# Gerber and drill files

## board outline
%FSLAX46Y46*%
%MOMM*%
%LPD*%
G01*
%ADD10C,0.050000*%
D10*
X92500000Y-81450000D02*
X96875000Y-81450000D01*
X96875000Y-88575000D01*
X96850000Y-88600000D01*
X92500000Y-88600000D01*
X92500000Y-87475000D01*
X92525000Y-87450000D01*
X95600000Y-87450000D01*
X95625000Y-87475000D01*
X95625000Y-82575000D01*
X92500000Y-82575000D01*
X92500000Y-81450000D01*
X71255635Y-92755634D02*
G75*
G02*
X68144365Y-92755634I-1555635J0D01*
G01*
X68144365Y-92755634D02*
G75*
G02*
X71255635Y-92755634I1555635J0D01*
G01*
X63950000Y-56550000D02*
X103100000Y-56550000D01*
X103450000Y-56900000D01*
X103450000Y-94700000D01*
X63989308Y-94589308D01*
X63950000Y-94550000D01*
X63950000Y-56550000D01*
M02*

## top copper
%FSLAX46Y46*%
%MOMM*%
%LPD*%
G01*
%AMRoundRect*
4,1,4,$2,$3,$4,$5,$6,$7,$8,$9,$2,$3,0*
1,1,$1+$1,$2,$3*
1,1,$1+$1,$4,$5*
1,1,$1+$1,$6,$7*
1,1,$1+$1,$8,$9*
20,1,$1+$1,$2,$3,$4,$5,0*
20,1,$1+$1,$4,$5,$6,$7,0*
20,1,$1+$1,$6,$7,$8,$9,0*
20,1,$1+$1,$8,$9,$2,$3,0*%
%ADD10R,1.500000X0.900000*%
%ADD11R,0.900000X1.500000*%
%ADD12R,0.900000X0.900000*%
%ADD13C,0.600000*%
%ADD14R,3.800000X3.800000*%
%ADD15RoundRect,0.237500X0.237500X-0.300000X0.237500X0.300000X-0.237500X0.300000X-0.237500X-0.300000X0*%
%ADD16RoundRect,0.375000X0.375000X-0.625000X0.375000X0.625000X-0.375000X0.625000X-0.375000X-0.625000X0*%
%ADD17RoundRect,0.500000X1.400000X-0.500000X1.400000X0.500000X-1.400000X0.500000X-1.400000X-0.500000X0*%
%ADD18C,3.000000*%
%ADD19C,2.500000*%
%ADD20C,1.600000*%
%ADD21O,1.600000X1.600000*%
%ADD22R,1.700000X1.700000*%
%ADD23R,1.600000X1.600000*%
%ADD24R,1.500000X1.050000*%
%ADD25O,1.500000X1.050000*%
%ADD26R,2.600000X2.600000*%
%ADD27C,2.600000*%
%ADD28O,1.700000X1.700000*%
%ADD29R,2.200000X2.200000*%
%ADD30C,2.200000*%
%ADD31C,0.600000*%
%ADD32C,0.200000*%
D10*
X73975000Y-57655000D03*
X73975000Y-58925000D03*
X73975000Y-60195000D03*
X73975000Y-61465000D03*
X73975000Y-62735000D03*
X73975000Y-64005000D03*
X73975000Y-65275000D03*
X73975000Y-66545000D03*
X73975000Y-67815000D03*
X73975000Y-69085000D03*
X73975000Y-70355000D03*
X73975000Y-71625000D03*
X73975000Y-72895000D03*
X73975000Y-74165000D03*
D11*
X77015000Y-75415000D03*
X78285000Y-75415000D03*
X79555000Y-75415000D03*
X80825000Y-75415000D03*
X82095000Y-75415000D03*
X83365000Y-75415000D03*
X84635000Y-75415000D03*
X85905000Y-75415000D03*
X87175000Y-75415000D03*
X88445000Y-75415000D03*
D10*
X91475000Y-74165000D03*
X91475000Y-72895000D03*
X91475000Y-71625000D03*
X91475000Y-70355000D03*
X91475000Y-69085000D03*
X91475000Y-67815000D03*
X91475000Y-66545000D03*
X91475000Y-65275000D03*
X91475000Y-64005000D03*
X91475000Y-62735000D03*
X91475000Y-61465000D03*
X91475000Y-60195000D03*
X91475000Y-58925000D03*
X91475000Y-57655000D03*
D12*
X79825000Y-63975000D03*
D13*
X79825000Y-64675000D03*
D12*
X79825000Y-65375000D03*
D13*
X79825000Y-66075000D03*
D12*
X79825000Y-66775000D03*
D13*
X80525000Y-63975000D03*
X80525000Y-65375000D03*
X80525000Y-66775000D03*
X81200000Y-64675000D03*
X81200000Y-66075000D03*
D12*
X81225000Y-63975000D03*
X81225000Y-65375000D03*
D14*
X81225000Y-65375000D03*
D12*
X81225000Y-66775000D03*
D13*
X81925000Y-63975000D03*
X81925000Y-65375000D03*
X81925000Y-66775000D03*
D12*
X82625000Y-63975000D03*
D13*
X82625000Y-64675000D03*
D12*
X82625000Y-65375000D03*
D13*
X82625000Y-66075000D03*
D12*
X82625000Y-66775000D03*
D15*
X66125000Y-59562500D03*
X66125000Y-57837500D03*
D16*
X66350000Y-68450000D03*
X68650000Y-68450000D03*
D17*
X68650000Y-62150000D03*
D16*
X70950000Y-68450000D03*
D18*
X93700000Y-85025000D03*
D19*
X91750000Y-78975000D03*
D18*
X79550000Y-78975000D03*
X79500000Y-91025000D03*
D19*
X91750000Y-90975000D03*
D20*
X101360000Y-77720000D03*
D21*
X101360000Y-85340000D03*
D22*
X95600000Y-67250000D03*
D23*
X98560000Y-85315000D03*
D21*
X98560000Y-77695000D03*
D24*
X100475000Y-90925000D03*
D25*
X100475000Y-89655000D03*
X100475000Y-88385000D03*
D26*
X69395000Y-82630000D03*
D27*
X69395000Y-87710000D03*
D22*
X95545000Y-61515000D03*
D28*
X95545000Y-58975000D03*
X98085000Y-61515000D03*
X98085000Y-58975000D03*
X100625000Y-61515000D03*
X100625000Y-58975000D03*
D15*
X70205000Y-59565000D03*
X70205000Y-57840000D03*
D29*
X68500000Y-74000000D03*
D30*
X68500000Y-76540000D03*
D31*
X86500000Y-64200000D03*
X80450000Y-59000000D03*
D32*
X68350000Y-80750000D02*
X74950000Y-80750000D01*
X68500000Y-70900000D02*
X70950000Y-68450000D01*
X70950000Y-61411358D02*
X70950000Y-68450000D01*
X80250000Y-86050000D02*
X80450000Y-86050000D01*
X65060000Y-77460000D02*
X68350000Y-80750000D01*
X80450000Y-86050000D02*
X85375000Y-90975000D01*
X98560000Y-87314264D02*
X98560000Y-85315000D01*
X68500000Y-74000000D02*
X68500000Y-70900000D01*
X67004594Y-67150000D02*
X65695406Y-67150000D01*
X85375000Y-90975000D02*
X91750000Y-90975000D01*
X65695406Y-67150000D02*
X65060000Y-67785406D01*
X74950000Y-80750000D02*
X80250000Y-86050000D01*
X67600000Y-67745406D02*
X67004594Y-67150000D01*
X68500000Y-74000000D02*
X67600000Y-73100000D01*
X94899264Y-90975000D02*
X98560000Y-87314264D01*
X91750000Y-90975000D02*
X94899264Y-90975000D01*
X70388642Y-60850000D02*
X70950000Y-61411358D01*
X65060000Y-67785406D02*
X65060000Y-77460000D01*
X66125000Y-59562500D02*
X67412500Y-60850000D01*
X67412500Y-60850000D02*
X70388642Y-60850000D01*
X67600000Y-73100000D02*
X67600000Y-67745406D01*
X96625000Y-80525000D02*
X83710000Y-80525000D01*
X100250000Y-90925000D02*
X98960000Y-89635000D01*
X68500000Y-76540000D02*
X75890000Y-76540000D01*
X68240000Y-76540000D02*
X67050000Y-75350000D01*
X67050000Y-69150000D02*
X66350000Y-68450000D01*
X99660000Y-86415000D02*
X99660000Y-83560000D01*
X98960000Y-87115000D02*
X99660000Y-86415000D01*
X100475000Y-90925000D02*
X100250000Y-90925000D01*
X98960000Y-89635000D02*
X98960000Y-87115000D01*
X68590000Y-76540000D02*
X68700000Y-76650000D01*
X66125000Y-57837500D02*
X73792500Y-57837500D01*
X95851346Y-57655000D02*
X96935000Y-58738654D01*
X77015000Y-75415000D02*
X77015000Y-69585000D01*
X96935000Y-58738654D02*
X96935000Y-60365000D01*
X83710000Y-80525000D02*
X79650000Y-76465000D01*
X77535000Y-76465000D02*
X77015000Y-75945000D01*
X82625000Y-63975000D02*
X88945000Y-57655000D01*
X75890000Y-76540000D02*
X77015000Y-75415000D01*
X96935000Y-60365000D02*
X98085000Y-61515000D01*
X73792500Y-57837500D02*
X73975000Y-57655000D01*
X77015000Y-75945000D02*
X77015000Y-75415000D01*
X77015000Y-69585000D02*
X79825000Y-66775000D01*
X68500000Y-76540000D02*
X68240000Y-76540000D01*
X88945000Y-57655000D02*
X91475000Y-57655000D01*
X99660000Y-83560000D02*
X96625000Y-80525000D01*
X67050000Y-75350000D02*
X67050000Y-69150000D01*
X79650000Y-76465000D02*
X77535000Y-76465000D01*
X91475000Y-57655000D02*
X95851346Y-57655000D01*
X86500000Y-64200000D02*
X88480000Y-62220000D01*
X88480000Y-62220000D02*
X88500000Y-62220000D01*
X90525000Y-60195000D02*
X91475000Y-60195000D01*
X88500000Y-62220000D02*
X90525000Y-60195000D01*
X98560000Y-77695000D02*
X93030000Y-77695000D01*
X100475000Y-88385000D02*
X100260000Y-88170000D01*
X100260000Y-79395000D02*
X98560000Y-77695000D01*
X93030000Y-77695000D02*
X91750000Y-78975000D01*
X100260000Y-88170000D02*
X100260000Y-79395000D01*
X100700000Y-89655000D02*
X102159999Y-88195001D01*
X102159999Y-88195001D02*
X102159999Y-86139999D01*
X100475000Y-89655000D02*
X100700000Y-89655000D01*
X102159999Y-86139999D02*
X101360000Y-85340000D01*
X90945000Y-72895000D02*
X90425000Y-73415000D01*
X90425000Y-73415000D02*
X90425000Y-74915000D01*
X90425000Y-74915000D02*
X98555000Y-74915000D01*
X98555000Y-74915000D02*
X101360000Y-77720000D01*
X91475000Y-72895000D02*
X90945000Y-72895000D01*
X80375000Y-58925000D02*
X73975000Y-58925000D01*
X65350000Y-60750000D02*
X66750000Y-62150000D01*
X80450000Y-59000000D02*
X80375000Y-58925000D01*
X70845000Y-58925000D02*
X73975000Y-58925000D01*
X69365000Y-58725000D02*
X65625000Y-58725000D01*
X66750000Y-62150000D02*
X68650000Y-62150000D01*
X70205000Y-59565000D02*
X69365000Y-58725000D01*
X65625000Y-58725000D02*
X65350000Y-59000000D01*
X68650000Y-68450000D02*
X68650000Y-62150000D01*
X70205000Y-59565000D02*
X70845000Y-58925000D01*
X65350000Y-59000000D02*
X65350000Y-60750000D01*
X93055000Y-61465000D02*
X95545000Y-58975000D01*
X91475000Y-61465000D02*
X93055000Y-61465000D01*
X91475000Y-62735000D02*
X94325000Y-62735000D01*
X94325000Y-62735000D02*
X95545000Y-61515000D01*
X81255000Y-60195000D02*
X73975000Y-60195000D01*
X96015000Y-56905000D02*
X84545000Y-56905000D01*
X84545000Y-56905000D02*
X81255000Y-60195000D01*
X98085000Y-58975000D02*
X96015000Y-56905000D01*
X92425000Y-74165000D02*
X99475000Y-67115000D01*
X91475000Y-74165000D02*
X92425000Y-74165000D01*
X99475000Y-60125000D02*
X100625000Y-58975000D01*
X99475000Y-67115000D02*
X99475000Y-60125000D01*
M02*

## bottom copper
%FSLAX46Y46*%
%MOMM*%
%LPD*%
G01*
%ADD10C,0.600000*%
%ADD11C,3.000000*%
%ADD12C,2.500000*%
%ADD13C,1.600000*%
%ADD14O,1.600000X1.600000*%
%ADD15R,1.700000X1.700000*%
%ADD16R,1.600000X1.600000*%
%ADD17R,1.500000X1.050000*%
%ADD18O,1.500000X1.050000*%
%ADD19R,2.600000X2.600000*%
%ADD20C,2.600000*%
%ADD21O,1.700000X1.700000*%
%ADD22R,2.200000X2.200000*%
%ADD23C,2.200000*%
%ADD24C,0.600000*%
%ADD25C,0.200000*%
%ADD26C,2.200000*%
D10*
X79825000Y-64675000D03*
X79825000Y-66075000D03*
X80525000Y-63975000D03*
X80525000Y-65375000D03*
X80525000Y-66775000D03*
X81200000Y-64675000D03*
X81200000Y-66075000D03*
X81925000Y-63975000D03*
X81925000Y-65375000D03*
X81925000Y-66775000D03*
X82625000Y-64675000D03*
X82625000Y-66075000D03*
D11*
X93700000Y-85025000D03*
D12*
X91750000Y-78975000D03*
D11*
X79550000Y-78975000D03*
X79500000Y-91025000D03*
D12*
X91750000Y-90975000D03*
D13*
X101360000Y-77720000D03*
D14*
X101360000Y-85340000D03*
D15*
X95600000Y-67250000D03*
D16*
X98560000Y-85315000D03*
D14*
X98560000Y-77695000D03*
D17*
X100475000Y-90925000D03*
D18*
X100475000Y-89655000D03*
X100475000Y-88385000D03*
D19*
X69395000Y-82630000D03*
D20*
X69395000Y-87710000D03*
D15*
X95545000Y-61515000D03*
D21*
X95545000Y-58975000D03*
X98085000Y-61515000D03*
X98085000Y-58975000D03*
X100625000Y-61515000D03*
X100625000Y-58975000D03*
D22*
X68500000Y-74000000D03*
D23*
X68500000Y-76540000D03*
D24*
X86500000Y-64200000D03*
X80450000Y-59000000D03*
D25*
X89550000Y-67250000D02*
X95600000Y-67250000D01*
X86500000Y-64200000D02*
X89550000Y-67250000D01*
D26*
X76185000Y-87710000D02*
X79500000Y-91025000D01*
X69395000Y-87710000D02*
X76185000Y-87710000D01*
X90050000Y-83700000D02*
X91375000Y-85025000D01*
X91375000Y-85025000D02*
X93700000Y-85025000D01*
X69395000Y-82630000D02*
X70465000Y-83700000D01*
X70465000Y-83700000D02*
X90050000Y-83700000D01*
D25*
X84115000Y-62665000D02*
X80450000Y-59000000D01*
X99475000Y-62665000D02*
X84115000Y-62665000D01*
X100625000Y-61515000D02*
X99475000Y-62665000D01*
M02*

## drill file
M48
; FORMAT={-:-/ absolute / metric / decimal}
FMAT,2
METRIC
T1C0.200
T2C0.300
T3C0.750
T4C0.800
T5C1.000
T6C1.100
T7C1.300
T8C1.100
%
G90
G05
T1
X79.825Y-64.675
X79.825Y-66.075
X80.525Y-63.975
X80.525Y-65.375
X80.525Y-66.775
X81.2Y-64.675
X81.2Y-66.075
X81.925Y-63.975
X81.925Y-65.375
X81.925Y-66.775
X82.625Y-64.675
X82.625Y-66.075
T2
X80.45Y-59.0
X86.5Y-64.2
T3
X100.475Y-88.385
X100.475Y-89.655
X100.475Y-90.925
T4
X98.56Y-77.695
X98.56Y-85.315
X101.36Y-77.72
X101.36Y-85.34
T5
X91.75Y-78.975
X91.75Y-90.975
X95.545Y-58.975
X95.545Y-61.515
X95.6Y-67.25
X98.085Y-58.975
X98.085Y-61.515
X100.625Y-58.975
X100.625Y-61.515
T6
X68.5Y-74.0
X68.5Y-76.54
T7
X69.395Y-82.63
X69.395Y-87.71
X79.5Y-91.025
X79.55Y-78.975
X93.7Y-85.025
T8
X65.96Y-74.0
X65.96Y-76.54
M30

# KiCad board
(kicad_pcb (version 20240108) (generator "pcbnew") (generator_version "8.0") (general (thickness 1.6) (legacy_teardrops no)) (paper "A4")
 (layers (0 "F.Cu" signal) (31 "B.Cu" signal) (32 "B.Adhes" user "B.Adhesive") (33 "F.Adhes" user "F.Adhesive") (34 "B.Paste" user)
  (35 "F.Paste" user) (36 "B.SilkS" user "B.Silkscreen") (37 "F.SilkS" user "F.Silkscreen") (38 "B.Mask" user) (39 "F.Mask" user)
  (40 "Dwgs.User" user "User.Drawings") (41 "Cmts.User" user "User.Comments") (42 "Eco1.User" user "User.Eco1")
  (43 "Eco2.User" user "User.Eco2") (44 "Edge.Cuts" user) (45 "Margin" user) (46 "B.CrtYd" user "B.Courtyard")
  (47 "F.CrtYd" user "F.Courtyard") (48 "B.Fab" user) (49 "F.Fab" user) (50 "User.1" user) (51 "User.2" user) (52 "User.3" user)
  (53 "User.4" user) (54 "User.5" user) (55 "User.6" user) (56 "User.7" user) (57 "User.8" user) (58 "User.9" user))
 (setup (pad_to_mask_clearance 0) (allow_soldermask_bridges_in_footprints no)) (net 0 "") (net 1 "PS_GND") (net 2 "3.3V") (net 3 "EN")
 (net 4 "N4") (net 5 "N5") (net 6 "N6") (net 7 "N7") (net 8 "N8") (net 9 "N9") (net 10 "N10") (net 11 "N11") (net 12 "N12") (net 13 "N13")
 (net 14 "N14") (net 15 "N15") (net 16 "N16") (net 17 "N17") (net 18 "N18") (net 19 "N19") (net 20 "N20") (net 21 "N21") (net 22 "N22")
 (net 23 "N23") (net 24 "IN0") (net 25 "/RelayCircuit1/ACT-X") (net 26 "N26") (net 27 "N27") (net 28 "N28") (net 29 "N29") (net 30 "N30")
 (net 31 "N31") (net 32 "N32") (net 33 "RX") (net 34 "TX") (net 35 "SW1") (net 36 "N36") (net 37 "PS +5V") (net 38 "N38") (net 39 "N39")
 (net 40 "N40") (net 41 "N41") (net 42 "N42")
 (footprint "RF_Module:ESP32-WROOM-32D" (layer "F.Cu") (at 82.725 65.905)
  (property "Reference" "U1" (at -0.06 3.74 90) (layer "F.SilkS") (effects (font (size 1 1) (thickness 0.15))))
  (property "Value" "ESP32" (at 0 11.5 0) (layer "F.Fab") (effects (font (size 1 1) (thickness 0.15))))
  (pad "1" smd rect (at -8.75 -8.25) (size 1.5 0.9) (layers "F.Cu" "F.Paste" "F.Mask") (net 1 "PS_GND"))
  (pad "2" smd rect (at -8.75 -6.98) (size 1.5 0.9) (layers "F.Cu" "F.Paste" "F.Mask") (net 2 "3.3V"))
  (pad "3" smd rect (at -8.75 -5.71) (size 1.5 0.9) (layers "F.Cu" "F.Paste" "F.Mask") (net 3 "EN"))
  (pad "4" smd rect (at -8.75 -4.44) (size 1.5 0.9) (layers "F.Cu" "F.Paste" "F.Mask") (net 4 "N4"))
  (pad "5" smd rect (at -8.75 -3.17) (size 1.5 0.9) (layers "F.Cu" "F.Paste" "F.Mask") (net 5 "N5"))
  (pad "6" smd rect (at -8.75 -1.9) (size 1.5 0.9) (layers "F.Cu" "F.Paste" "F.Mask") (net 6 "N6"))
  (pad "7" smd rect (at -8.75 -0.63) (size 1.5 0.9) (layers "F.Cu" "F.Paste" "F.Mask") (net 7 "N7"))
  (pad "8" smd rect (at -8.75 0.64) (size 1.5 0.9) (layers "F.Cu" "F.Paste" "F.Mask") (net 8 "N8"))
  (pad "9" smd rect (at -8.75 1.91) (size 1.5 0.9) (layers "F.Cu" "F.Paste" "F.Mask") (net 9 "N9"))
  (pad "10" smd rect (at -8.75 3.18) (size 1.5 0.9) (layers "F.Cu" "F.Paste" "F.Mask") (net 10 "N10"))
  (pad "11" smd rect (at -8.75 4.45) (size 1.5 0.9) (layers "F.Cu" "F.Paste" "F.Mask") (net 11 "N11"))
  (pad "12" smd rect (at -8.75 5.72) (size 1.5 0.9) (layers "F.Cu" "F.Paste" "F.Mask") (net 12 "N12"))
  (pad "13" smd rect (at -8.75 6.99) (size 1.5 0.9) (layers "F.Cu" "F.Paste" "F.Mask") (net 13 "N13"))
  (pad "14" smd rect (at -8.75 8.26) (size 1.5 0.9) (layers "F.Cu" "F.Paste" "F.Mask") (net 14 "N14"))
  (pad "15" smd rect (at -5.71 9.51 90) (size 1.5 0.9) (layers "F.Cu" "F.Paste" "F.Mask") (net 1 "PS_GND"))
  (pad "16" smd rect (at -4.44 9.51 90) (size 1.5 0.9) (layers "F.Cu" "F.Paste" "F.Mask") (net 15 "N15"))
  (pad "17" smd rect (at -3.17 9.51 90) (size 1.5 0.9) (layers "F.Cu" "F.Paste" "F.Mask") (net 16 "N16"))
  (pad "18" smd rect (at -1.9 9.51 90) (size 1.5 0.9) (layers "F.Cu" "F.Paste" "F.Mask") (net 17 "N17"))
  (pad "19" smd rect (at -0.63 9.51 90) (size 1.5 0.9) (layers "F.Cu" "F.Paste" "F.Mask") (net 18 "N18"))
  (pad "20" smd rect (at 0.64 9.51 90) (size 1.5 0.9) (layers "F.Cu" "F.Paste" "F.Mask") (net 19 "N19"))
  (pad "21" smd rect (at 1.91 9.51 90) (size 1.5 0.9) (layers "F.Cu" "F.Paste" "F.Mask") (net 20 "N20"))
  (pad "22" smd rect (at 3.18 9.51 90) (size 1.5 0.9) (layers "F.Cu" "F.Paste" "F.Mask") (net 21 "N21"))
  (pad "23" smd rect (at 4.45 9.51 90) (size 1.5 0.9) (layers "F.Cu" "F.Paste" "F.Mask") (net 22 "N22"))
  (pad "24" smd rect (at 5.72 9.51 90) (size 1.5 0.9) (layers "F.Cu" "F.Paste" "F.Mask") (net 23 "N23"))
  (pad "25" smd rect (at 8.75 8.26) (size 1.5 0.9) (layers "F.Cu" "F.Paste" "F.Mask") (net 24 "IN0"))
  (pad "26" smd rect (at 8.75 6.99) (size 1.5 0.9) (layers "F.Cu" "F.Paste" "F.Mask") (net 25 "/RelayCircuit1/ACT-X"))
  (pad "27" smd rect (at 8.75 5.72) (size 1.5 0.9) (layers "F.Cu" "F.Paste" "F.Mask") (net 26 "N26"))
  (pad "28" smd rect (at 8.75 4.45) (size 1.5 0.9) (layers "F.Cu" "F.Paste" "F.Mask") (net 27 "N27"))
  (pad "29" smd rect (at 8.75 3.18) (size 1.5 0.9) (layers "F.Cu" "F.Paste" "F.Mask") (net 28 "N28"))
  (pad "30" smd rect (at 8.75 1.91) (size 1.5 0.9) (layers "F.Cu" "F.Paste" "F.Mask") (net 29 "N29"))
  (pad "31" smd rect (at 8.75 0.64) (size 1.5 0.9) (layers "F.Cu" "F.Paste" "F.Mask") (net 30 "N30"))
  (pad "32" smd rect (at 8.75 -0.63) (size 1.5 0.9) (layers "F.Cu" "F.Paste" "F.Mask") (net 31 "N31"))
  (pad "33" smd rect (at 8.75 -1.9) (size 1.5 0.9) (layers "F.Cu" "F.Paste" "F.Mask") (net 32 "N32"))
  (pad "34" smd rect (at 8.75 -3.17) (size 1.5 0.9) (layers "F.Cu" "F.Paste" "F.Mask") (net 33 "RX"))
  (pad "35" smd rect (at 8.75 -4.44) (size 1.5 0.9) (layers "F.Cu" "F.Paste" "F.Mask") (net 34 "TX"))
  (pad "36" smd rect (at 8.75 -5.71) (size 1.5 0.9) (layers "F.Cu" "F.Paste" "F.Mask") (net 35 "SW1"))
  (pad "37" smd rect (at 8.75 -6.98) (size 1.5 0.9) (layers "F.Cu" "F.Paste" "F.Mask") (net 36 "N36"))
  (pad "38" smd rect (at 8.75 -8.25) (size 1.5 0.9) (layers "F.Cu" "F.Paste" "F.Mask") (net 1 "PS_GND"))
  (pad "39" smd rect (at -2.9 -1.93) (size 0.9 0.9) (layers "F.Cu" "F.Paste") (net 1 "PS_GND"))
  (pad "39" thru_hole circle (at -2.9 -1.23) (size 0.6 0.6) (drill 0.2) (layers "*.Cu" "F.Mask") (remove_unused_layers no) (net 1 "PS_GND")
   (zone_connect 2))
  (pad "39" smd rect (at -2.9 -0.53) (size 0.9 0.9) (layers "F.Cu" "F.Paste") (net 1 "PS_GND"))
  (pad "39" thru_hole circle (at -2.9 0.17) (size 0.6 0.6) (drill 0.2) (layers "*.Cu" "F.Mask") (remove_unused_layers no) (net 1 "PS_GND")
   (zone_connect 2))
  (pad "39" smd rect (at -2.9 0.87) (size 0.9 0.9) (layers "F.Cu" "F.Paste") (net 1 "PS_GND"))
  (pad "39" thru_hole circle (at -2.2 -1.93) (size 0.6 0.6) (drill 0.2) (layers "*.Cu" "F.Mask") (remove_unused_layers no) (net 1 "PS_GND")
   (zone_connect 2))
  (pad "39" thru_hole circle (at -2.2 -0.53) (size 0.6 0.6) (drill 0.2) (layers "*.Cu" "F.Mask") (remove_unused_layers no) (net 1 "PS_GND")
   (zone_connect 2))
  (pad "39" thru_hole circle (at -2.2 0.87) (size 0.6 0.6) (drill 0.2) (layers "*.Cu" "F.Mask") (remove_unused_layers no) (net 1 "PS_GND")
   (zone_connect 2))
  (pad "39" thru_hole circle (at -1.525 -1.23) (size 0.6 0.6) (drill 0.2) (layers "*.Cu" "F.Mask") (remove_unused_layers no)
   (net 1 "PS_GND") (zone_connect 2))
  (pad "39" thru_hole circle (at -1.525 0.17) (size 0.6 0.6) (drill 0.2) (layers "*.Cu" "F.Mask") (remove_unused_layers no) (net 1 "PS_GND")
   (zone_connect 2))
  (pad "39" smd rect (at -1.5 -1.93) (size 0.9 0.9) (layers "F.Cu" "F.Paste") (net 1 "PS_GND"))
  (pad "39" smd rect (at -1.5 -0.53) (size 0.9 0.9) (layers "F.Cu" "F.Paste") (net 1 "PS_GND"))
  (pad "39" smd rect (at -1.5 -0.53) (size 3.8 3.8) (layers "F.Cu" "F.Mask") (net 1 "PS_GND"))
  (pad "39" smd rect (at -1.5 0.87) (size 0.9 0.9) (layers "F.Cu" "F.Paste") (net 1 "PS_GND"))
  (pad "39" thru_hole circle (at -0.8 -1.93) (size 0.6 0.6) (drill 0.2) (layers "*.Cu" "F.Mask") (remove_unused_layers no) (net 1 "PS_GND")
   (zone_connect 2))
  (pad "39" thru_hole circle (at -0.8 -0.53) (size 0.6 0.6) (drill 0.2) (layers "*.Cu" "F.Mask") (remove_unused_layers no) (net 1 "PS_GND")
   (zone_connect 2))
  (pad "39" thru_hole circle (at -0.8 0.87) (size 0.6 0.6) (drill 0.2) (layers "*.Cu" "F.Mask") (remove_unused_layers no) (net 1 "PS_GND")
   (zone_connect 2))
  (pad "39" smd rect (at -0.1 -1.93) (size 0.9 0.9) (layers "F.Cu" "F.Paste") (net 1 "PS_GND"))
  (pad "39" thru_hole circle (at -0.1 -1.23) (size 0.6 0.6) (drill 0.2) (layers "*.Cu" "F.Mask") (remove_unused_layers no) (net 1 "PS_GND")
   (zone_connect 2))
  (pad "39" smd rect (at -0.1 -0.53) (size 0.9 0.9) (layers "F.Cu" "F.Paste") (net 1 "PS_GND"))
  (pad "39" thru_hole circle (at -0.1 0.17) (size 0.6 0.6) (drill 0.2) (layers "*.Cu" "F.Mask") (remove_unused_layers no) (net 1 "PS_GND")
   (zone_connect 2))
  (pad "39" smd rect (at -0.1 0.87) (size 0.9 0.9) (layers "F.Cu" "F.Paste") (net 1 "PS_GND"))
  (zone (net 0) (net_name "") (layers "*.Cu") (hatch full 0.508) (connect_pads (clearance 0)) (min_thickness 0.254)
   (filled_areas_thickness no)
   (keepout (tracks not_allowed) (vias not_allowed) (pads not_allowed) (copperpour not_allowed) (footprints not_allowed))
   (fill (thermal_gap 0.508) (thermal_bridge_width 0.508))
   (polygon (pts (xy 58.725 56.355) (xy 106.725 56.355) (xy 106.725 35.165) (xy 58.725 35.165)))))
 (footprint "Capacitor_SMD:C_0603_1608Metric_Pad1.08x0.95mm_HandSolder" (layer "F.Cu") (at 66.125 58.7 90)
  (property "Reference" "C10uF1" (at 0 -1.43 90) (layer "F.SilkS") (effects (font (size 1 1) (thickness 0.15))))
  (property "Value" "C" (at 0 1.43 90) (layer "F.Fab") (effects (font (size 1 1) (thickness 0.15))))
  (pad "1" smd roundrect (at -0.8625 0 90) (size 1.075 0.95) (layers "F.Cu" "F.Paste" "F.Mask") (roundrect_rratio 0.25) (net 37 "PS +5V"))
  (pad "2" smd roundrect (at 0.8625 0 90) (size 1.075 0.95) (layers "F.Cu" "F.Paste" "F.Mask") (roundrect_rratio 0.25) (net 1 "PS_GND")))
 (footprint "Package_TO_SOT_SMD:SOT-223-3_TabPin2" (layer "F.Cu") (at 68.65 65.3 90)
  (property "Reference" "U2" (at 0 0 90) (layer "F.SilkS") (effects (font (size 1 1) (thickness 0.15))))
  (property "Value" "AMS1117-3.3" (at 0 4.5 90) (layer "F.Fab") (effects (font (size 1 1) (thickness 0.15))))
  (pad "1" smd roundrect (at -3.15 -2.3 90) (size 2 1.5) (layers "F.Cu" "F.Paste" "F.Mask") (roundrect_rratio 0.25) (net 1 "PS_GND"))
  (pad "2" smd roundrect (at -3.15 0 90) (size 2 1.5) (layers "F.Cu" "F.Paste" "F.Mask") (roundrect_rratio 0.25) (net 2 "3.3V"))
  (pad "2" smd roundrect (at 3.15 0 90) (size 2 3.8) (layers "F.Cu" "F.Paste" "F.Mask") (roundrect_rratio 0.25) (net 2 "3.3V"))
  (pad "3" smd roundrect (at -3.15 2.3 90) (size 2 1.5) (layers "F.Cu" "F.Paste" "F.Mask") (roundrect_rratio 0.25) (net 37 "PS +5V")))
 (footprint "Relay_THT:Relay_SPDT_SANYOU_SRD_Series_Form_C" (layer "F.Cu") (at 93.7 85.025 180)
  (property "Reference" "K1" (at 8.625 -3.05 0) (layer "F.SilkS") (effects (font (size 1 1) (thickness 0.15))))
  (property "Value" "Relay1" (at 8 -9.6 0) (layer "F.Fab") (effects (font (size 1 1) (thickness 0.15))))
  (pad "1" thru_hole circle (at 0 0 270) (size 3 3) (drill 1.3) (layers "*.Cu" "*.Mask") (remove_unused_layers no) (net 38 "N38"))
  (pad "2" thru_hole circle (at 1.95 6.05 270) (size 2.5 2.5) (drill 1) (layers "*.Cu" "*.Mask") (remove_unused_layers no) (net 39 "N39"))
  (pad "3" thru_hole circle (at 14.15 6.05 270) (size 3 3) (drill 1.3) (layers "*.Cu" "*.Mask") (remove_unused_layers no) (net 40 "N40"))
  (pad "4" thru_hole circle (at 14.2 -6 270) (size 3 3) (drill 1.3) (layers "*.Cu" "*.Mask") (remove_unused_layers no) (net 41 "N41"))
  (pad "5" thru_hole circle (at 1.95 -5.95 270) (size 2.5 2.5) (drill 1) (layers "*.Cu" "*.Mask") (remove_unused_layers no)
   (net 37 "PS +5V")))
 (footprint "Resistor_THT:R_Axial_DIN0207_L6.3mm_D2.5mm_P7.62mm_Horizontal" (layer "F.Cu") (at 101.36 77.72 -90)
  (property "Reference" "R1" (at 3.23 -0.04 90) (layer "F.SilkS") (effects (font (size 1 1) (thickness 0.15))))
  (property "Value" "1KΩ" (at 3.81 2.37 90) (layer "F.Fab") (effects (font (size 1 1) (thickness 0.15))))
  (pad "1" thru_hole circle (at 0 0 270) (size 1.6 1.6) (drill 0.8) (layers "*.Cu" "*.Mask") (remove_unused_layers no)
   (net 25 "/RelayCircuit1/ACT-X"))
  (pad "2" thru_hole oval (at 7.62 0 270) (size 1.6 1.6) (drill 0.8) (layers "*.Cu" "*.Mask") (remove_unused_layers no) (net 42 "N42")))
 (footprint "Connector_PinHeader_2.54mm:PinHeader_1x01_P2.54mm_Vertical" (layer "F.Cu") (at 95.6 67.25)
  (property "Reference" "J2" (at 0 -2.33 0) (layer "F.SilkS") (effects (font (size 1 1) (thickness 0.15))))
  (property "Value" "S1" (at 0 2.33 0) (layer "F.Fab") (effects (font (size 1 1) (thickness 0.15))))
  (pad "1" thru_hole rect (at 0 0) (size 1.7 1.7) (drill 1) (layers "*.Cu" "*.Mask") (remove_unused_layers no) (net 35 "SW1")))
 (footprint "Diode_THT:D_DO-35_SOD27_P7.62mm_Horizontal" (layer "F.Cu") (at 98.56 85.315 90)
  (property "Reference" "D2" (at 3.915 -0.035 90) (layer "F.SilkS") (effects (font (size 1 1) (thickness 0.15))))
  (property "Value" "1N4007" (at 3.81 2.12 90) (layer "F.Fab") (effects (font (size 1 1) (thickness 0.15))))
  (pad "1" thru_hole rect (at 0 0 90) (size 1.6 1.6) (drill 0.8) (layers "*.Cu" "*.Mask") (remove_unused_layers no) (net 37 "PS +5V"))
  (pad "2" thru_hole oval (at 7.62 0 90) (size 1.6 1.6) (drill 0.8) (layers "*.Cu" "*.Mask") (remove_unused_layers no) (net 39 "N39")))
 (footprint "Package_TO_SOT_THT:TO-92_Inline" (layer "F.Cu") (at 100.475 90.925 90)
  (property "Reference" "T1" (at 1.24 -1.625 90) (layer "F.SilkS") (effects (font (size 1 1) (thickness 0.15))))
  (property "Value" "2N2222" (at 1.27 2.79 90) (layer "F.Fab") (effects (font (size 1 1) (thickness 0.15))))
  (pad "1" thru_hole rect (at 0 0 90) (size 1.05 1.5) (drill 0.75) (layers "*.Cu" "*.Mask") (remove_unused_layers no) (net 1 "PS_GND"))
  (pad "2" thru_hole oval (at 1.27 0 90) (size 1.05 1.5) (drill 0.75) (layers "*.Cu" "*.Mask") (remove_unused_layers no) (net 42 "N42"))
  (pad "3" thru_hole oval (at 2.54 0 90) (size 1.05 1.5) (drill 0.75) (layers "*.Cu" "*.Mask") (remove_unused_layers no) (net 39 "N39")))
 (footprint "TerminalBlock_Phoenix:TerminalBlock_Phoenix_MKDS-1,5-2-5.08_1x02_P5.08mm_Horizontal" (layer "F.Cu") (at 69.395 82.63 -90)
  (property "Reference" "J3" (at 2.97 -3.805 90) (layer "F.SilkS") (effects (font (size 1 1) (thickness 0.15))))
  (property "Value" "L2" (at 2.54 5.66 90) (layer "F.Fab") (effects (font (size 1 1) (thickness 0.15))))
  (pad "1" thru_hole rect (at 0 0 270) (size 2.6 2.6) (drill 1.3) (layers "*.Cu" "*.Mask") (remove_unused_layers no) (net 38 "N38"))
  (pad "2" thru_hole circle (at 5.08 0 270) (size 2.6 2.6) (drill 1.3) (layers "*.Cu" "*.Mask") (remove_unused_layers no) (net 41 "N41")))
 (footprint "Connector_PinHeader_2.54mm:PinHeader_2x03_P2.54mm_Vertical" (layer "F.Cu") (at 95.545 61.515 90)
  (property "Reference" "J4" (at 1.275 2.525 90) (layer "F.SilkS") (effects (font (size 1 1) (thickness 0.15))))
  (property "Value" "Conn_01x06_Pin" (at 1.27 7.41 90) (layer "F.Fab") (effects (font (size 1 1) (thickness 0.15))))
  (pad "1" thru_hole rect (at 0 0 90) (size 1.7 1.7) (drill 1) (layers "*.Cu" "*.Mask") (remove_unused_layers no) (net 33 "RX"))
  (pad "2" thru_hole oval (at 2.54 0 90) (size 1.7 1.7) (drill 1) (layers "*.Cu" "*.Mask") (remove_unused_layers no) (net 34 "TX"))
  (pad "3" thru_hole oval (at 0 2.54 90) (size 1.7 1.7) (drill 1) (layers "*.Cu" "*.Mask") (remove_unused_layers no) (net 1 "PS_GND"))
  (pad "4" thru_hole oval (at 2.54 2.54 90) (size 1.7 1.7) (drill 1) (layers "*.Cu" "*.Mask") (remove_unused_layers no) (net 3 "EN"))
  (pad "5" thru_hole oval (at 0 5.08 90) (size 1.7 1.7) (drill 1) (layers "*.Cu" "*.Mask") (remove_unused_layers no) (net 2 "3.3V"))
  (pad "6" thru_hole oval (at 2.54 5.08 90) (size 1.7 1.7) (drill 1) (layers "*.Cu" "*.Mask") (remove_unused_layers no) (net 24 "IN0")))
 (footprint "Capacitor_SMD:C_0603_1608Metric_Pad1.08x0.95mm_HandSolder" (layer "F.Cu") (at 70.205 58.7025 90)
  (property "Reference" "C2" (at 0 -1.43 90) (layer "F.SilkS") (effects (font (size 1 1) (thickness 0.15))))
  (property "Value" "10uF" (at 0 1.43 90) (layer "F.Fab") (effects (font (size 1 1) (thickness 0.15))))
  (pad "1" smd roundrect (at -0.8625 0 90) (size 1.075 0.95) (layers "F.Cu" "F.Paste" "F.Mask") (roundrect_rratio 0.25) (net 2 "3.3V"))
  (pad "2" smd roundrect (at 0.8625 0 90) (size 1.075 0.95) (layers "F.Cu" "F.Paste" "F.Mask") (roundrect_rratio 0.25) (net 1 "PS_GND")))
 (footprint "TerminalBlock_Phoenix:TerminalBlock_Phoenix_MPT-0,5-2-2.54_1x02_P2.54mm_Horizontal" (layer "F.Cu") (at 68.5 74 -90)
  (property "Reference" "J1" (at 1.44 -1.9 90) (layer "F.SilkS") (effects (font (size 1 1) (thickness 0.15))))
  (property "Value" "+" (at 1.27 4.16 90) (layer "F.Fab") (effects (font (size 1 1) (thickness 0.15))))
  (pad "" np_thru_hole circle (at 0 2.54 270) (size 1.1 1.1) (drill 1.1) (layers "*.Cu" "*.Mask"))
  (pad "" np_thru_hole circle (at 2.54 2.54 270) (size 1.1 1.1) (drill 1.1) (layers "*.Cu" "*.Mask"))
  (pad "1" thru_hole rect (at 0 0 270) (size 2.2 2.2) (drill 1.1) (layers "*.Cu" "*.Mask") (remove_unused_layers no) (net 37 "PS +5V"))
  (pad "2" thru_hole circle (at 2.54 0 270) (size 2.2 2.2) (drill 1.1) (layers "*.Cu" "*.Mask") (remove_unused_layers no) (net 1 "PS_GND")))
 (gr_poly
  (pts (xy 92.5 81.45) (xy 96.875 81.45) (xy 96.875 88.575) (xy 96.85 88.6) (xy 92.5 88.6) (xy 92.5 87.475) (xy 92.525 87.45)
   (xy 95.6 87.45) (xy 95.625 87.475) (xy 95.625 82.575) (xy 92.5 82.575))
  (stroke (width 0.05) (type solid)) (fill none) (layer "Edge.Cuts"))
 (gr_circle (center 69.7 92.755634) (end 70.8 93.855634) (stroke (width 0.05) (type default)) (fill none) (layer "Edge.Cuts"))
 (gr_poly
  (pts (xy 63.95 56.55) (xy 103.1 56.55) (xy 103.45 56.9) (xy 103.45 94.7) (xy 63.989308 94.589308) (xy 63.95 94.55))
  (stroke (width 0.05) (type solid)) (fill none) (layer "Edge.Cuts"))
 (segment (start 68.35 80.75) (end 74.95 80.75) (width 0.2) (layer "F.Cu") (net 37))
 (segment (start 68.5 70.9) (end 70.95 68.45) (width 0.2) (layer "F.Cu") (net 37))
 (segment (start 70.95 61.411358) (end 70.95 68.45) (width 0.2) (layer "F.Cu") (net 37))
 (segment (start 80.25 86.05) (end 80.45 86.05) (width 0.2) (layer "F.Cu") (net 37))
 (segment (start 65.06 77.46) (end 68.35 80.75) (width 0.2) (layer "F.Cu") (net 37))
 (segment (start 80.45 86.05) (end 85.375 90.975) (width 0.2) (layer "F.Cu") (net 37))
 (segment (start 98.56 87.314264) (end 98.56 85.315) (width 0.2) (layer "F.Cu") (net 37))
 (segment (start 68.5 74) (end 68.5 70.9) (width 0.2) (layer "F.Cu") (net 37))
 (segment (start 67.004594 67.15) (end 65.695406 67.15) (width 0.2) (layer "F.Cu") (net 37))
 (segment (start 85.375 90.975) (end 91.75 90.975) (width 0.2) (layer "F.Cu") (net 37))
 (segment (start 65.695406 67.15) (end 65.06 67.785406) (width 0.2) (layer "F.Cu") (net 37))
 (segment (start 74.95 80.75) (end 80.25 86.05) (width 0.2) (layer "F.Cu") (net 37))
 (segment (start 67.6 67.745406) (end 67.004594 67.15) (width 0.2) (layer "F.Cu") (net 37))
 (segment (start 68.5 74) (end 67.6 73.1) (width 0.2) (layer "F.Cu") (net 37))
 (segment (start 94.899264 90.975) (end 98.56 87.314264) (width 0.2) (layer "F.Cu") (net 37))
 (segment (start 91.75 90.975) (end 94.899264 90.975) (width 0.2) (layer "F.Cu") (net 37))
 (segment (start 70.388642 60.85) (end 70.95 61.411358) (width 0.2) (layer "F.Cu") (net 37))
 (segment (start 65.06 67.785406) (end 65.06 77.46) (width 0.2) (layer "F.Cu") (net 37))
 (segment (start 66.125 59.5625) (end 67.4125 60.85) (width 0.2) (layer "F.Cu") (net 37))
 (segment (start 67.4125 60.85) (end 70.388642 60.85) (width 0.2) (layer "F.Cu") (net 37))
 (segment (start 67.6 73.1) (end 67.6 67.745406) (width 0.2) (layer "F.Cu") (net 37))
 (segment (start 96.625 80.525) (end 83.71 80.525) (width 0.2) (layer "F.Cu") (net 1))
 (segment (start 100.25 90.925) (end 98.96 89.635) (width 0.2) (layer "F.Cu") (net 1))
 (segment (start 68.5 76.54) (end 75.89 76.54) (width 0.2) (layer "F.Cu") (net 1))
 (segment (start 68.24 76.54) (end 67.05 75.35) (width 0.2) (layer "F.Cu") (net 1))
 (segment (start 67.05 69.15) (end 66.35 68.45) (width 0.2) (layer "F.Cu") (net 1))
 (segment (start 99.66 86.415) (end 99.66 83.56) (width 0.2) (layer "F.Cu") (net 1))
 (segment (start 98.96 87.115) (end 99.66 86.415) (width 0.2) (layer "F.Cu") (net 1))
 (segment (start 100.475 90.925) (end 100.25 90.925) (width 0.2) (layer "F.Cu") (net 1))
 (segment (start 98.96 89.635) (end 98.96 87.115) (width 0.2) (layer "F.Cu") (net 1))
 (segment (start 68.59 76.54) (end 68.7 76.65) (width 0.2) (layer "F.Cu") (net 1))
 (segment (start 66.125 57.8375) (end 73.7925 57.8375) (width 0.2) (layer "F.Cu") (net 1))
 (segment (start 95.851346 57.655) (end 96.935 58.738654) (width 0.2) (layer "F.Cu") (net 1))
 (segment (start 77.015 75.415) (end 77.015 69.585) (width 0.2) (layer "F.Cu") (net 1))
 (segment (start 96.935 58.738654) (end 96.935 60.365) (width 0.2) (layer "F.Cu") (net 1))
 (segment (start 83.71 80.525) (end 79.65 76.465) (width 0.2) (layer "F.Cu") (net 1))
 (segment (start 77.535 76.465) (end 77.015 75.945) (width 0.2) (layer "F.Cu") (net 1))
 (segment (start 82.625 63.975) (end 88.945 57.655) (width 0.2) (layer "F.Cu") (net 1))
 (segment (start 75.89 76.54) (end 77.015 75.415) (width 0.2) (layer "F.Cu") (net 1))
 (segment (start 96.935 60.365) (end 98.085 61.515) (width 0.2) (layer "F.Cu") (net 1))
 (segment (start 73.7925 57.8375) (end 73.975 57.655) (width 0.2) (layer "F.Cu") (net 1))
 (segment (start 77.015 75.945) (end 77.015 75.415) (width 0.2) (layer "F.Cu") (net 1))
 (segment (start 77.015 69.585) (end 79.825 66.775) (width 0.2) (layer "F.Cu") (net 1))
 (segment (start 68.5 76.54) (end 68.24 76.54) (width 0.2) (layer "F.Cu") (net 1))
 (segment (start 88.945 57.655) (end 91.475 57.655) (width 0.2) (layer "F.Cu") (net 1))
 (segment (start 99.66 83.56) (end 96.625 80.525) (width 0.2) (layer "F.Cu") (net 1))
 (segment (start 67.05 75.35) (end 67.05 69.15) (width 0.2) (layer "F.Cu") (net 1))
 (segment (start 79.65 76.465) (end 77.535 76.465) (width 0.2) (layer "F.Cu") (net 1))
 (segment (start 91.475 57.655) (end 95.851346 57.655) (width 0.2) (layer "F.Cu") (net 1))
 (segment (start 86.5 64.2) (end 88.48 62.22) (width 0.2) (layer "F.Cu") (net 35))
 (segment (start 88.48 62.22) (end 88.5 62.22) (width 0.2) (layer "F.Cu") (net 35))
 (segment (start 90.525 60.195) (end 91.475 60.195) (width 0.2) (layer "F.Cu") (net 35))
 (segment (start 88.5 62.22) (end 90.525 60.195) (width 0.2) (layer "F.Cu") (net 35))
 (via (at 86.5 64.2) (size 0.6) (drill 0.3) (layers "F.Cu" "B.Cu") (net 35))
 (segment (start 89.55 67.25) (end 95.6 67.25) (width 0.2) (layer "B.Cu") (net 35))
 (segment (start 86.5 64.2) (end 89.55 67.25) (width 0.2) (layer "B.Cu") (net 35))
 (segment (start 98.56 77.695) (end 93.03 77.695) (width 0.2) (layer "F.Cu") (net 39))
 (segment (start 100.475 88.385) (end 100.26 88.17) (width 0.2) (layer "F.Cu") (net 39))
 (segment (start 100.26 79.395) (end 98.56 77.695) (width 0.2) (layer "F.Cu") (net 39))
 (segment (start 93.03 77.695) (end 91.75 78.975) (width 0.2) (layer "F.Cu") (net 39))
 (segment (start 100.26 88.17) (end 100.26 79.395) (width 0.2) (layer "F.Cu") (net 39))
 (segment (start 100.7 89.655) (end 102.159999 88.195001) (width 0.2) (layer "F.Cu") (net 42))
 (segment (start 102.159999 88.195001) (end 102.159999 86.139999) (width 0.2) (layer "F.Cu") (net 42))
 (segment (start 100.475 89.655) (end 100.7 89.655) (width 0.2) (layer "F.Cu") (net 42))
 (segment (start 102.159999 86.139999) (end 101.36 85.34) (width 0.2) (layer "F.Cu") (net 42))
 (segment (start 90.945 72.895) (end 90.425 73.415) (width 0.2) (layer "F.Cu") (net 25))
 (segment (start 90.425 73.415) (end 90.425 74.915) (width 0.2) (layer "F.Cu") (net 25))
 (segment (start 90.425 74.915) (end 98.555 74.915) (width 0.2) (layer "F.Cu") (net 25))
 (segment (start 98.555 74.915) (end 101.36 77.72) (width 0.2) (layer "F.Cu") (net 25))
 (segment (start 91.475 72.895) (end 90.945 72.895) (width 0.2) (layer "F.Cu") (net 25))
 (segment (start 76.185 87.71) (end 79.5 91.025) (width 2.2) (layer "B.Cu") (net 41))
 (segment (start 69.395 87.71) (end 76.185 87.71) (width 2.2) (layer "B.Cu") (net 41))
 (segment (start 90.05 83.7) (end 91.375 85.025) (width 2.2) (layer "B.Cu") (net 38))
 (segment (start 91.375 85.025) (end 93.7 85.025) (width 2.2) (layer "B.Cu") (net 38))
 (segment (start 69.395 82.63) (end 70.465 83.7) (width 2.2) (layer "B.Cu") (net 38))
 (segment (start 70.465 83.7) (end 90.05 83.7) (width 2.2) (layer "B.Cu") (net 38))
 (segment (start 80.375 58.925) (end 73.975 58.925) (width 0.2) (layer "F.Cu") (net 2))
 (segment (start 65.35 60.75) (end 66.75 62.15) (width 0.2) (layer "F.Cu") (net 2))
 (segment (start 80.45 59) (end 80.375 58.925) (width 0.2) (layer "F.Cu") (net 2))
 (segment (start 70.845 58.925) (end 73.975 58.925) (width 0.2) (layer "F.Cu") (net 2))
 (segment (start 69.365 58.725) (end 65.625 58.725) (width 0.2) (layer "F.Cu") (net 2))
 (segment (start 66.75 62.15) (end 68.65 62.15) (width 0.2) (layer "F.Cu") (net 2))
 (segment (start 70.205 59.565) (end 69.365 58.725) (width 0.2) (layer "F.Cu") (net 2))
 (segment (start 65.625 58.725) (end 65.35 59) (width 0.2) (layer "F.Cu") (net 2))
 (segment (start 68.65 68.45) (end 68.65 62.15) (width 0.2) (layer "F.Cu") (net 2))
 (segment (start 70.205 59.565) (end 70.845 58.925) (width 0.2) (layer "F.Cu") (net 2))
 (segment (start 65.35 59) (end 65.35 60.75) (width 0.2) (layer "F.Cu") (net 2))
 (via (at 80.45 59) (size 0.6) (drill 0.3) (layers "F.Cu" "B.Cu") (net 2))
 (segment (start 84.115 62.665) (end 80.45 59) (width 0.2) (layer "B.Cu") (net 2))
 (segment (start 99.475 62.665) (end 84.115 62.665) (width 0.2) (layer "B.Cu") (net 2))
 (segment (start 100.625 61.515) (end 99.475 62.665) (width 0.2) (layer "B.Cu") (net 2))
 (segment (start 93.055 61.465) (end 95.545 58.975) (width 0.2) (layer "F.Cu") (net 34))
 (segment (start 91.475 61.465) (end 93.055 61.465) (width 0.2) (layer "F.Cu") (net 34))
 (segment (start 91.475 62.735) (end 94.325 62.735) (width 0.2) (layer "F.Cu") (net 33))
 (segment (start 94.325 62.735) (end 95.545 61.515) (width 0.2) (layer "F.Cu") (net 33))
 (segment (start 81.255 60.195) (end 73.975 60.195) (width 0.2) (layer "F.Cu") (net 3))
 (segment (start 96.015 56.905) (end 84.545 56.905) (width 0.2) (layer "F.Cu") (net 3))
 (segment (start 84.545 56.905) (end 81.255 60.195) (width 0.2) (layer "F.Cu") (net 3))
 (segment (start 98.085 58.975) (end 96.015 56.905) (width 0.2) (layer "F.Cu") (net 3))
 (segment (start 92.425 74.165) (end 99.475 67.115) (width 0.2) (layer "F.Cu") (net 24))
 (segment (start 91.475 74.165) (end 92.425 74.165) (width 0.2) (layer "F.Cu") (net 24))
 (segment (start 99.475 60.125) (end 100.625 58.975) (width 0.2) (layer "F.Cu") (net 24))
 (segment (start 99.475 67.115) (end 99.475 60.125) (width 0.2) (layer "F.Cu") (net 24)))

